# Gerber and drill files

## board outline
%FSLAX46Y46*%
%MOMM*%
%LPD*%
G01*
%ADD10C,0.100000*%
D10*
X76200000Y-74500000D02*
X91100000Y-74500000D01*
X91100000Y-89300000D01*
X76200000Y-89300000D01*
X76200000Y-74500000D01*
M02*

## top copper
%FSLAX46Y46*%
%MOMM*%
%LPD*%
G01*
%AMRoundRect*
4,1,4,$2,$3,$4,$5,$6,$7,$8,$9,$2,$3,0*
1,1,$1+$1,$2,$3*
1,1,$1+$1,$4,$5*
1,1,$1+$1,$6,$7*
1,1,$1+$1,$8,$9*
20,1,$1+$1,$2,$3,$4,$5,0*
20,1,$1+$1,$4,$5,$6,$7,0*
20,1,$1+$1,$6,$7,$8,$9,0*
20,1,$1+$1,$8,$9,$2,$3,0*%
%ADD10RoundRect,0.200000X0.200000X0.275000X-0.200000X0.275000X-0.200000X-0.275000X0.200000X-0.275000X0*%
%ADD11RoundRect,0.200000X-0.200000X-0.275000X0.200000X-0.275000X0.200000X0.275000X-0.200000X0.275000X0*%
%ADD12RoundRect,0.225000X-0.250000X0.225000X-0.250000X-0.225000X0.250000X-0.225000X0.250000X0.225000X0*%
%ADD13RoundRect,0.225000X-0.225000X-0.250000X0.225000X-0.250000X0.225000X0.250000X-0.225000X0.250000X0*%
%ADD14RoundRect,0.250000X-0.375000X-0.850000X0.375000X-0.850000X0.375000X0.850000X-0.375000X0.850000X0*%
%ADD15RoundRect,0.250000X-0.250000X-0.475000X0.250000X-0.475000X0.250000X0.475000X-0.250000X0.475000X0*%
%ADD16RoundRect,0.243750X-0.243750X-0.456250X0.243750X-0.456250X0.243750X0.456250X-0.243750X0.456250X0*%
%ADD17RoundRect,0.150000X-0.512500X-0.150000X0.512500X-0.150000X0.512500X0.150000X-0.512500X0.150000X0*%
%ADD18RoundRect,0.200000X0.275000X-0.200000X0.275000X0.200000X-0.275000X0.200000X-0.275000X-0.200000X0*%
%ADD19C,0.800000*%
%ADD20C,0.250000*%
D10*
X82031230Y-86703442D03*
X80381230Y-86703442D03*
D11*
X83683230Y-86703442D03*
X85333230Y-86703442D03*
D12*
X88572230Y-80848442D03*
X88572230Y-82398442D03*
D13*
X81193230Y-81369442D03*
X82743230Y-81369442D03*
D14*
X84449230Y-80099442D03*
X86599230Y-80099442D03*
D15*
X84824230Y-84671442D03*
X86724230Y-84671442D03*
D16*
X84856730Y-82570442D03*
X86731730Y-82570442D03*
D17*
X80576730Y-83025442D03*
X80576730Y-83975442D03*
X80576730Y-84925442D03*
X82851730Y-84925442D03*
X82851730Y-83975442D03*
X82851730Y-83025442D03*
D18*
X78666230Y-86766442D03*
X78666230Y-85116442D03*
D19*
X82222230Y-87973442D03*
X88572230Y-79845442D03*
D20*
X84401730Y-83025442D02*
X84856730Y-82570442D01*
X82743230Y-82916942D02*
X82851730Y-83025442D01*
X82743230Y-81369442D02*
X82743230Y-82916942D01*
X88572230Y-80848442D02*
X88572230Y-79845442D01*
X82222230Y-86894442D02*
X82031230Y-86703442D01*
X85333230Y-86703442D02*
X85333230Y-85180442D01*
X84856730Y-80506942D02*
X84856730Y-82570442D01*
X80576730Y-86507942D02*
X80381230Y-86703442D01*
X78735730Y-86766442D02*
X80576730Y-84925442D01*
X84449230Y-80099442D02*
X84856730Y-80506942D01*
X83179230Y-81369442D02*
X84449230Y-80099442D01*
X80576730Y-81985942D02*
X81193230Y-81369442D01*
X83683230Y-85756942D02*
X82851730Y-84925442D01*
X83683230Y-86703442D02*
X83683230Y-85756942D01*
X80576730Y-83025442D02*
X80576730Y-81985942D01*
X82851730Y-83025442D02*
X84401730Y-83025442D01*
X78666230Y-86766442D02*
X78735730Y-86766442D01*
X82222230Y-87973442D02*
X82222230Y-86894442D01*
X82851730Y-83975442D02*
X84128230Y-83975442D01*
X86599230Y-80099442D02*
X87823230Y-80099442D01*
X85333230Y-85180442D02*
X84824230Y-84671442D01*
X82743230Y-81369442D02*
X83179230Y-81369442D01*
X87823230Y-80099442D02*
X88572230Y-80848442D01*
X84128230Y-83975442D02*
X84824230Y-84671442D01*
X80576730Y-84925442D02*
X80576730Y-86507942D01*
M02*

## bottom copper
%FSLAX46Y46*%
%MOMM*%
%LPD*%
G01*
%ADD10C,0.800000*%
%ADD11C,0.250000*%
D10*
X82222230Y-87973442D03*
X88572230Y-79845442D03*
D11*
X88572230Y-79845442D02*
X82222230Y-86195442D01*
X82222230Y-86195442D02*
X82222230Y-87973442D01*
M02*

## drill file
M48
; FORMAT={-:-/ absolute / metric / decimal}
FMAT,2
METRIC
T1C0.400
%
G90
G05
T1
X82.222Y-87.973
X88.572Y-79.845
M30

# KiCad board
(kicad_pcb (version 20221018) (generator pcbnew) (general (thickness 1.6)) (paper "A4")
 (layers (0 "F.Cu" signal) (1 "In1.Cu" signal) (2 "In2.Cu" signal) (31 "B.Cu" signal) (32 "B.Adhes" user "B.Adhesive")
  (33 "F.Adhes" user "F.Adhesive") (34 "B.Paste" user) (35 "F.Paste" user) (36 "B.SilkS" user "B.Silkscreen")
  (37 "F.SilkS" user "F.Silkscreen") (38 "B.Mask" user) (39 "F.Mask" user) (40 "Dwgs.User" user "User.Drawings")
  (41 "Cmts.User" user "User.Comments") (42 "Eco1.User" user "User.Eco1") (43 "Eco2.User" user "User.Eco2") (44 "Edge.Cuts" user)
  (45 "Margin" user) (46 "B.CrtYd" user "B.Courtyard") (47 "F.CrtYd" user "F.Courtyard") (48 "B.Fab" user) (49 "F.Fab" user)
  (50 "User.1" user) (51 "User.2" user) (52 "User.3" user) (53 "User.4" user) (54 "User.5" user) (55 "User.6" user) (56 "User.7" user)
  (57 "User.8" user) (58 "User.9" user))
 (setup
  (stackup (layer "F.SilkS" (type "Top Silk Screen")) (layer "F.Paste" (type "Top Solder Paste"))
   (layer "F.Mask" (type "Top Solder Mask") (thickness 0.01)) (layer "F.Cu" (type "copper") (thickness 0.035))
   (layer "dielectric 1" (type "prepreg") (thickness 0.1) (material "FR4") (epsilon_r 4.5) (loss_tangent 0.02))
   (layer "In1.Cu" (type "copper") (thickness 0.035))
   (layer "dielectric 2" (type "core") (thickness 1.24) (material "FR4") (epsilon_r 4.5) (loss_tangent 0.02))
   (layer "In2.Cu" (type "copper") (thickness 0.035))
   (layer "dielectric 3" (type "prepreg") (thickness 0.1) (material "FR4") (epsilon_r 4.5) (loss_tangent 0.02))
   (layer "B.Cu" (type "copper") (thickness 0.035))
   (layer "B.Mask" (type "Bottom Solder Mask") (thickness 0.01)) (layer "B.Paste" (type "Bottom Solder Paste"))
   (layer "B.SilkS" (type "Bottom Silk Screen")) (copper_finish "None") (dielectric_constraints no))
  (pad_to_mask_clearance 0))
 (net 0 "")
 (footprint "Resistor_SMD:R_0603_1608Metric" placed (layer "F.Cu") (at 81.20623 86.703442 180)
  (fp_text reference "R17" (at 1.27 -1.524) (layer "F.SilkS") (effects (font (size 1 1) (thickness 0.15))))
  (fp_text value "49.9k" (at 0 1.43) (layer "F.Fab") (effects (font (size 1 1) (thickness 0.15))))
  (pad "1" smd roundrect (at -0.825 0 180) (size 0.8 0.95) (layers "F.Cu" "F.Paste" "F.Mask") (roundrect_rratio 0.25))
  (pad "2" smd roundrect (at 0.825 0 180) (size 0.8 0.95) (layers "F.Cu" "F.Paste" "F.Mask") (roundrect_rratio 0.25)))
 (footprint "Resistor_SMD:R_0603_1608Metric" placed (layer "F.Cu") (at 84.50823 86.703442)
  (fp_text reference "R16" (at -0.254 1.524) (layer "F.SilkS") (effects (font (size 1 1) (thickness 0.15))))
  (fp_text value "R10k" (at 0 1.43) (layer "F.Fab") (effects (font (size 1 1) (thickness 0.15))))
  (pad "1" smd roundrect (at -0.825 0) (size 0.8 0.95) (layers "F.Cu" "F.Paste" "F.Mask") (roundrect_rratio 0.25))
  (pad "2" smd roundrect (at 0.825 0) (size 0.8 0.95) (layers "F.Cu" "F.Paste" "F.Mask") (roundrect_rratio 0.25)))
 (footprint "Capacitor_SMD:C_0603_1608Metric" (layer "F.Cu") (at 88.57223 81.623442 -90)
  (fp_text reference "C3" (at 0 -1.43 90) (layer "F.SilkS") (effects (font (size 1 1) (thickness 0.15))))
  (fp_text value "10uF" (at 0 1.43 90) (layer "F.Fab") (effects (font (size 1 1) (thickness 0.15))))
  (pad "1" smd roundrect (at -0.775 0 270) (size 0.9 0.95) (layers "F.Cu" "F.Paste" "F.Mask") (roundrect_rratio 0.25))
  (pad "2" smd roundrect (at 0.775 0 270) (size 0.9 0.95) (layers "F.Cu" "F.Paste" "F.Mask") (roundrect_rratio 0.25)))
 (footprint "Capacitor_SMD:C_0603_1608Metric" (layer "F.Cu") (at 81.96823 81.369442)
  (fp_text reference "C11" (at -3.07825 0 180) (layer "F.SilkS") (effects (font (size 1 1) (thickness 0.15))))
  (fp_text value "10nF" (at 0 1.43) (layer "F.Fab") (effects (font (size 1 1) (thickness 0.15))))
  (pad "1" smd roundrect (at -0.775 0) (size 0.9 0.95) (layers "F.Cu" "F.Paste" "F.Mask") (roundrect_rratio 0.25))
  (pad "2" smd roundrect (at 0.775 0) (size 0.9 0.95) (layers "F.Cu" "F.Paste" "F.Mask") (roundrect_rratio 0.25)))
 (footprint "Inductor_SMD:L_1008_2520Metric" (layer "F.Cu") (at 85.52423 80.099442)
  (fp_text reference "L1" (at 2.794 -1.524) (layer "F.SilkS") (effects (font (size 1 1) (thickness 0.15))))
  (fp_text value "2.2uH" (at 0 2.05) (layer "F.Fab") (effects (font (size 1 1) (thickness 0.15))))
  (pad "1" smd roundrect (at -1.075 0) (size 1.25 2.2) (layers "F.Cu" "F.Paste" "F.Mask") (roundrect_rratio 0.2))
  (pad "2" smd roundrect (at 1.075 0) (size 1.25 2.2) (layers "F.Cu" "F.Paste" "F.Mask") (roundrect_rratio 0.2)))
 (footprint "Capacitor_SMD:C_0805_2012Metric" (layer "F.Cu") (at 85.77423 84.671442)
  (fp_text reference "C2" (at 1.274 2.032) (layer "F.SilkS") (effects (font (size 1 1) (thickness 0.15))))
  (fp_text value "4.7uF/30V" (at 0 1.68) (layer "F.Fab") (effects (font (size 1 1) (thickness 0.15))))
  (pad "1" smd roundrect (at -0.95 0) (size 1 1.45) (layers "F.Cu" "F.Paste" "F.Mask") (roundrect_rratio 0.25))
  (pad "2" smd roundrect (at 0.95 0) (size 1 1.45) (layers "F.Cu" "F.Paste" "F.Mask") (roundrect_rratio 0.25)))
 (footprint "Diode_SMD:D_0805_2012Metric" (layer "F.Cu") (at 85.79423 82.570442)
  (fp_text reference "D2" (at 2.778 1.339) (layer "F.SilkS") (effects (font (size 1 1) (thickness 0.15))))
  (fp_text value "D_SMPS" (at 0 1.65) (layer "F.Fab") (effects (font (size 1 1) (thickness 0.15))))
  (pad "1" smd roundrect (at -0.9375 0) (size 0.975 1.4) (layers "F.Cu" "F.Paste" "F.Mask") (roundrect_rratio 0.25))
  (pad "2" smd roundrect (at 0.9375 0) (size 0.975 1.4) (layers "F.Cu" "F.Paste" "F.Mask") (roundrect_rratio 0.25)))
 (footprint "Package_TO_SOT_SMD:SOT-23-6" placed (layer "F.Cu") (at 81.71423 83.975442)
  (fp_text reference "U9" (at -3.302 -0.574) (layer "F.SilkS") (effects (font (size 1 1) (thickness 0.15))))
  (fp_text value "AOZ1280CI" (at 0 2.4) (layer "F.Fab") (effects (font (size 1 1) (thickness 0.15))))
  (pad "1" smd roundrect (at -1.1375 -0.95) (size 1.325 0.6) (layers "F.Cu" "F.Paste" "F.Mask") (roundrect_rratio 0.25))
  (pad "2" smd roundrect (at -1.1375 0) (size 1.325 0.6) (layers "F.Cu" "F.Paste" "F.Mask") (roundrect_rratio 0.25))
  (pad "3" smd roundrect (at -1.1375 0.95) (size 1.325 0.6) (layers "F.Cu" "F.Paste" "F.Mask") (roundrect_rratio 0.25))
  (pad "4" smd roundrect (at 1.1375 0.95) (size 1.325 0.6) (layers "F.Cu" "F.Paste" "F.Mask") (roundrect_rratio 0.25))
  (pad "5" smd roundrect (at 1.1375 0) (size 1.325 0.6) (layers "F.Cu" "F.Paste" "F.Mask") (roundrect_rratio 0.25))
  (pad "6" smd roundrect (at 1.1375 -0.95) (size 1.325 0.6) (layers "F.Cu" "F.Paste" "F.Mask") (roundrect_rratio 0.25)))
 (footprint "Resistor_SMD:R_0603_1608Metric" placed (layer "F.Cu") (at 78.66623 85.941442 90)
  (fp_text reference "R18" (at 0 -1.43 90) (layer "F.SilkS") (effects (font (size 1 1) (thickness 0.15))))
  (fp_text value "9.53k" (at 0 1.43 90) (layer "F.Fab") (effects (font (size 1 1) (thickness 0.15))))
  (pad "1" smd roundrect (at -0.825 0 90) (size 0.8 0.95) (layers "F.Cu" "F.Paste" "F.Mask") (roundrect_rratio 0.25))
  (pad "2" smd roundrect (at 0.825 0 90) (size 0.8 0.95) (layers "F.Cu" "F.Paste" "F.Mask") (roundrect_rratio 0.25)))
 (gr_rect (start 76.2 74.5) (end 91.1 89.3) (stroke (width 0.1) (type default)) (fill none) (layer "Edge.Cuts"))
 (segment (start 84.40173 83.025442) (end 84.85673 82.570442) (width 0.25) (layer "F.Cu") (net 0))
 (segment (start 82.74323 82.916942) (end 82.85173 83.025442) (width 0.25) (layer "F.Cu") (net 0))
 (segment (start 82.74323 81.369442) (end 82.74323 82.916942) (width 0.25) (layer "F.Cu") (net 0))
 (segment (start 88.57223 80.848442) (end 88.57223 79.845442) (width 0.25) (layer "F.Cu") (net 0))
 (segment (start 82.22223 86.894442) (end 82.03123 86.703442) (width 0.25) (layer "F.Cu") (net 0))
 (segment (start 85.33323 86.703442) (end 85.33323 85.180442) (width 0.25) (layer "F.Cu") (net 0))
 (segment (start 84.85673 80.506942) (end 84.85673 82.570442) (width 0.25) (layer "F.Cu") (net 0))
 (segment (start 80.57673 86.507942) (end 80.38123 86.703442) (width 0.25) (layer "F.Cu") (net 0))
 (segment (start 78.73573 86.766442) (end 80.57673 84.925442) (width 0.25) (layer "F.Cu") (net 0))
 (segment (start 84.44923 80.099442) (end 84.85673 80.506942) (width 0.25) (layer "F.Cu") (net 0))
 (segment (start 83.17923 81.369442) (end 84.44923 80.099442) (width 0.25) (layer "F.Cu") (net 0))
 (segment (start 80.57673 81.985942) (end 81.19323 81.369442) (width 0.25) (layer "F.Cu") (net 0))
 (segment (start 83.68323 85.756942) (end 82.85173 84.925442) (width 0.25) (layer "F.Cu") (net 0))
 (segment (start 83.68323 86.703442) (end 83.68323 85.756942) (width 0.25) (layer "F.Cu") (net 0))
 (segment (start 80.57673 83.025442) (end 80.57673 81.985942) (width 0.25) (layer "F.Cu") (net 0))
 (segment (start 82.85173 83.025442) (end 84.40173 83.025442) (width 0.25) (layer "F.Cu") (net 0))
 (segment (start 78.66623 86.766442) (end 78.73573 86.766442) (width 0.25) (layer "F.Cu") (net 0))
 (segment (start 82.22223 87.973442) (end 82.22223 86.894442) (width 0.25) (layer "F.Cu") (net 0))
 (segment (start 82.85173 83.975442) (end 84.12823 83.975442) (width 0.25) (layer "F.Cu") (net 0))
 (segment (start 86.59923 80.099442) (end 87.82323 80.099442) (width 0.25) (layer "F.Cu") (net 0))
 (segment (start 85.33323 85.180442) (end 84.82423 84.671442) (width 0.25) (layer "F.Cu") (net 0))
 (segment (start 82.74323 81.369442) (end 83.17923 81.369442) (width 0.25) (layer "F.Cu") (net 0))
 (segment (start 87.82323 80.099442) (end 88.57223 80.848442) (width 0.25) (layer "F.Cu") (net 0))
 (segment (start 84.12823 83.975442) (end 84.82423 84.671442) (width 0.25) (layer "F.Cu") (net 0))
 (segment (start 80.57673 84.925442) (end 80.57673 86.507942) (width 0.25) (layer "F.Cu") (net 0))
 (via (at 82.22223 87.973442) (size 0.8) (drill 0.4) (layers "F.Cu" "B.Cu") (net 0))
 (via (at 88.57223 79.845442) (size 0.8) (drill 0.4) (layers "F.Cu" "B.Cu") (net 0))
 (segment (start 88.57223 79.845442) (end 82.22223 86.195442) (width 0.25) (layer "B.Cu") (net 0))
 (segment (start 82.22223 86.195442) (end 82.22223 87.973442) (width 0.25) (layer "B.Cu") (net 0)))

